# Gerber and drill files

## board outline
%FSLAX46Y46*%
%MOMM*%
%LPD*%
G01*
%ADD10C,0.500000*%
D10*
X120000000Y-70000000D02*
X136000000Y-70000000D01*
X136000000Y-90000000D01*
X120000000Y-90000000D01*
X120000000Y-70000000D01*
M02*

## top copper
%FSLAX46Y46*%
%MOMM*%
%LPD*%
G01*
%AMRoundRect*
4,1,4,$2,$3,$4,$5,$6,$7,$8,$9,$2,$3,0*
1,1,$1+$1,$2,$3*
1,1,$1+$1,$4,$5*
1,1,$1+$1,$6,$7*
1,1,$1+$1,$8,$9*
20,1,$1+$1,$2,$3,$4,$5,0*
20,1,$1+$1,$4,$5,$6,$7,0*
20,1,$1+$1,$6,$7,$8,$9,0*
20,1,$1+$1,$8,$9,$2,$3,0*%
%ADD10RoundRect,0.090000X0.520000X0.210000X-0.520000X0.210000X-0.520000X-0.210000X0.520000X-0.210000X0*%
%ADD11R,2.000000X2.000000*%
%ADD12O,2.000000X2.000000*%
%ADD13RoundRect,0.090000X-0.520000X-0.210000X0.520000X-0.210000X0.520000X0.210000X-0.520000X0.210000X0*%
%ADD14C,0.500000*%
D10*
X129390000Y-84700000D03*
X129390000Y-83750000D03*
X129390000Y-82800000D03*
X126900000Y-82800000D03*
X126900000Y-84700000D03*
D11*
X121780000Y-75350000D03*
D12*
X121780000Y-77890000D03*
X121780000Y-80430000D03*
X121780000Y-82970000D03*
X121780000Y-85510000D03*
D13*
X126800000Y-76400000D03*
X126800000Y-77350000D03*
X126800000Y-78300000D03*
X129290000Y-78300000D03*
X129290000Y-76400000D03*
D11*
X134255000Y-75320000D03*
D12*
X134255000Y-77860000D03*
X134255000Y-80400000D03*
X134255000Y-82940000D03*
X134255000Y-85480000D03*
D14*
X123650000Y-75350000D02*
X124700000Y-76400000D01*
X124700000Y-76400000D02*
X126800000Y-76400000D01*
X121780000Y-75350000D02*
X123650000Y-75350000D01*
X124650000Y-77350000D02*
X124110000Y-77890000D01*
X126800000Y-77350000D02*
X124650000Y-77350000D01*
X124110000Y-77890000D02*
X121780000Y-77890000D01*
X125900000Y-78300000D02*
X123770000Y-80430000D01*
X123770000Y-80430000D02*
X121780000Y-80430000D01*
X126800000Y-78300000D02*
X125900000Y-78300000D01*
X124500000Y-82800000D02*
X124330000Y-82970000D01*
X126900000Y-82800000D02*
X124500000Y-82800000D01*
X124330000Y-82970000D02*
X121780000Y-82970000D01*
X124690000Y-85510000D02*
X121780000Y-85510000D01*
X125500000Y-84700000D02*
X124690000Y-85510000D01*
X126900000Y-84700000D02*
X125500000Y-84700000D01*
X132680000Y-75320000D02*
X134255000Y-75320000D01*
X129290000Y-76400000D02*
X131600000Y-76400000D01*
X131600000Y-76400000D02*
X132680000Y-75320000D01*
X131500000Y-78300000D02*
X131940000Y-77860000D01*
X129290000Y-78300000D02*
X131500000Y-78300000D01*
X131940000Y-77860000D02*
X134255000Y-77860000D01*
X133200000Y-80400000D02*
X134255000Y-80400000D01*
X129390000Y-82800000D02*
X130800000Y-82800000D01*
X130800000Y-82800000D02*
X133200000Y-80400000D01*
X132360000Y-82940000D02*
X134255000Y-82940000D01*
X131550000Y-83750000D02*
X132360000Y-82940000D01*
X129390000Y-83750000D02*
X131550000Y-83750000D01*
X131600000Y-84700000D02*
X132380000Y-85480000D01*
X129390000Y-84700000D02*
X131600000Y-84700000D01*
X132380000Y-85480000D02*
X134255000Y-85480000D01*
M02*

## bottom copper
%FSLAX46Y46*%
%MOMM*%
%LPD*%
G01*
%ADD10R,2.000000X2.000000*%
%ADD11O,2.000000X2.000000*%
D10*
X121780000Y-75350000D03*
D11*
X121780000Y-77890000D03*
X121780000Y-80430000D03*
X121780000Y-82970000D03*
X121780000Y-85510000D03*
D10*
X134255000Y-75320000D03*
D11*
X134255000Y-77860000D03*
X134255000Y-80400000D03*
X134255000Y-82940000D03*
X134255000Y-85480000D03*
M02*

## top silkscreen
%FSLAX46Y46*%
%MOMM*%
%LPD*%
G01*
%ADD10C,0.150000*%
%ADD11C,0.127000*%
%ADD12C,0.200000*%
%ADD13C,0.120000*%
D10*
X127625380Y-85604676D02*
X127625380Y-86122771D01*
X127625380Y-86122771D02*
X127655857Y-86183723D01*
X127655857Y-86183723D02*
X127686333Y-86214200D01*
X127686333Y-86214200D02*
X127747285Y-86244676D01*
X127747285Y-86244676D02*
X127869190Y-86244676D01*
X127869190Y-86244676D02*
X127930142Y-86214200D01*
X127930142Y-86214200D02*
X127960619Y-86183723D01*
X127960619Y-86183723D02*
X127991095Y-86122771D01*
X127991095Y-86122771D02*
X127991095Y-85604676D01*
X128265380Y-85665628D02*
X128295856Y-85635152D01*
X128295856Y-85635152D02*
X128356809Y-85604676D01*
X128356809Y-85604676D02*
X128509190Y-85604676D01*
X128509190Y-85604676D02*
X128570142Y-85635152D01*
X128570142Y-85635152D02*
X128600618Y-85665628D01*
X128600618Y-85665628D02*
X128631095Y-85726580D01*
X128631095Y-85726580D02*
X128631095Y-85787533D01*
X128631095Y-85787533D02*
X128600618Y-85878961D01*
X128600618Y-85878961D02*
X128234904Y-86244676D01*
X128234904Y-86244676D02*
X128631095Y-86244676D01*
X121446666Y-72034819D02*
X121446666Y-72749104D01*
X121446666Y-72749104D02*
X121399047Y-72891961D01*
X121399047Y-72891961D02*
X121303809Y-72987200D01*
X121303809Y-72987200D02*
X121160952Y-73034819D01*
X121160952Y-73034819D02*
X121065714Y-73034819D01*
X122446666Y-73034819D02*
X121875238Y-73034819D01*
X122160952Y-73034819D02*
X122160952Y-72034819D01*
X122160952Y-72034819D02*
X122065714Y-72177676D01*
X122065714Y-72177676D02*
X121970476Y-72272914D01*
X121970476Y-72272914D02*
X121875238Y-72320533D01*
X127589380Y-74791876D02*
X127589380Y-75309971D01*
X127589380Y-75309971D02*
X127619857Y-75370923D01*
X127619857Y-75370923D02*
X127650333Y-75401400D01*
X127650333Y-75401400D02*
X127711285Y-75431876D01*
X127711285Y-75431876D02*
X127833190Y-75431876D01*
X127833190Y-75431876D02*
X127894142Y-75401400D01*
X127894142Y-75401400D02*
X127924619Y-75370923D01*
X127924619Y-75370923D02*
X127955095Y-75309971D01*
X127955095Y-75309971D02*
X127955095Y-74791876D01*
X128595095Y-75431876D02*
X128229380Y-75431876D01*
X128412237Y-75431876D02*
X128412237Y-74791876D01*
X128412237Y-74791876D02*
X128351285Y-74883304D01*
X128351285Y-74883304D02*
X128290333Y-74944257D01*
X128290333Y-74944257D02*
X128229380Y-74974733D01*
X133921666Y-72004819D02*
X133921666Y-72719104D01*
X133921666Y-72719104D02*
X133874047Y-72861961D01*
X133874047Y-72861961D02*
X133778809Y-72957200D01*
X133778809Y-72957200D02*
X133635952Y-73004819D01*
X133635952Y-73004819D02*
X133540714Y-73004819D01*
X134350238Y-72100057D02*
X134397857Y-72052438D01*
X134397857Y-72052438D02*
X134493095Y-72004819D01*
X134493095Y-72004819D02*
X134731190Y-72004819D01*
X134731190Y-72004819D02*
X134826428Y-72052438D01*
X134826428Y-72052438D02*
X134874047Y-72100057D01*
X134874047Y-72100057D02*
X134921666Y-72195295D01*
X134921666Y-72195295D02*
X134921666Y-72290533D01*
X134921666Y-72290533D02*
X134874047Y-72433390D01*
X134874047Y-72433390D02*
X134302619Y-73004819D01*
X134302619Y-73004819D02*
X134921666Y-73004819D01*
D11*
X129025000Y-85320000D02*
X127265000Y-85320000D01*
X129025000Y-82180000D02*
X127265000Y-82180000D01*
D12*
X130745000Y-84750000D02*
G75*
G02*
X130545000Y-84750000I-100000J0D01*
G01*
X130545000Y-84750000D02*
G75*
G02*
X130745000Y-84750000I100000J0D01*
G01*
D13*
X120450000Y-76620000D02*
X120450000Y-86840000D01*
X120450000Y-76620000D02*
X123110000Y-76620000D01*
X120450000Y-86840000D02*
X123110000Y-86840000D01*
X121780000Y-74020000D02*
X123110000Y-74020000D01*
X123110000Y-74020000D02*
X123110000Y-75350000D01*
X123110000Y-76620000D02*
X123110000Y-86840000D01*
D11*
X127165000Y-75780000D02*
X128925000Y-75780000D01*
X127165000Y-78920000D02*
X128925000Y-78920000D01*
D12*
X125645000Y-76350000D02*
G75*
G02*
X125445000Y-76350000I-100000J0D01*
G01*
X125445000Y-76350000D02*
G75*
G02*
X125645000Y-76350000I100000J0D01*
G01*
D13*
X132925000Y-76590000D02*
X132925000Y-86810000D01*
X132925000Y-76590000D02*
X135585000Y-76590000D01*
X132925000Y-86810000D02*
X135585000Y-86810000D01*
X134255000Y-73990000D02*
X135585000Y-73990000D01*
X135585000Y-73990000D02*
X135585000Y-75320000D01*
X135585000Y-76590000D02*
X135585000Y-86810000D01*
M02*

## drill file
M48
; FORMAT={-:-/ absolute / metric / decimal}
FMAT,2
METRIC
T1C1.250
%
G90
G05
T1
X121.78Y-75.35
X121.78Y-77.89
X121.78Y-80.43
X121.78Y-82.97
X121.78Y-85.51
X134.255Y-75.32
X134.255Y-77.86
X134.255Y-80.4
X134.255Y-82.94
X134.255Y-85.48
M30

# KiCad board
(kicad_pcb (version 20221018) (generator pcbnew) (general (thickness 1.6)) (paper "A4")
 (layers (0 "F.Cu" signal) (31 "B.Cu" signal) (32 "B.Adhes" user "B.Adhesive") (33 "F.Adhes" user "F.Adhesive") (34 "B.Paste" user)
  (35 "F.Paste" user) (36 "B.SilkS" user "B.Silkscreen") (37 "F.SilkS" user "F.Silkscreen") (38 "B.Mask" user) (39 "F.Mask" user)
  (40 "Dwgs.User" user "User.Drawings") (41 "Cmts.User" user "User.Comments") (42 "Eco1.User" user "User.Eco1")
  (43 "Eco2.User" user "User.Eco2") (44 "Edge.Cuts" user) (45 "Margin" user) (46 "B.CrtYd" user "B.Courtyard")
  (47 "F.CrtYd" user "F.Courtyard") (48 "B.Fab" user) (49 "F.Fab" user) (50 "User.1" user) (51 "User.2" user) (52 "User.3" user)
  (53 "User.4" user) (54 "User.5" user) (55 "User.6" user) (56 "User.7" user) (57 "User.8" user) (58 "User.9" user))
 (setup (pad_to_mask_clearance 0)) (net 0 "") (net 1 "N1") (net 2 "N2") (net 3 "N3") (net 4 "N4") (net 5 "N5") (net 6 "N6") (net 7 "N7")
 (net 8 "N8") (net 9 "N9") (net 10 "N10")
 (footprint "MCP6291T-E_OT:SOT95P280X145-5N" (layer "F.Cu") (at 128.145 83.75 180)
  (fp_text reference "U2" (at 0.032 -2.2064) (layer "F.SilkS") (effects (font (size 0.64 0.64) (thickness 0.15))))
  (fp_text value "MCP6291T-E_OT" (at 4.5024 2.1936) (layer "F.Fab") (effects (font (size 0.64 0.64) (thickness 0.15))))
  (fp_line (start -0.88 -1.57) (end 0.88 -1.57) (stroke (width 0.127) (type solid)) (layer "F.SilkS"))
  (fp_line (start -0.88 1.57) (end 0.88 1.57) (stroke (width 0.127) (type solid)) (layer "F.SilkS"))
  (fp_circle (center -2.5 -1) (end -2.4 -1) (stroke (width 0.2) (type solid)) (fill none) (layer "F.SilkS"))
  (pad "1" smd roundrect (at -1.245 -0.95 180) (size 1.22 0.6) (layers "F.Cu" "F.Paste" "F.Mask") (roundrect_rratio 0.15) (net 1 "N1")
   (solder_mask_margin 0.102))
  (pad "2" smd roundrect (at -1.245 0 180) (size 1.22 0.6) (layers "F.Cu" "F.Paste" "F.Mask") (roundrect_rratio 0.15) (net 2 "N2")
   (solder_mask_margin 0.102))
  (pad "3" smd roundrect (at -1.245 0.95 180) (size 1.22 0.6) (layers "F.Cu" "F.Paste" "F.Mask") (roundrect_rratio 0.15) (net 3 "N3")
   (solder_mask_margin 0.102))
  (pad "4" smd roundrect (at 1.245 0.95 180) (size 1.22 0.6) (layers "F.Cu" "F.Paste" "F.Mask") (roundrect_rratio 0.15) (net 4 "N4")
   (solder_mask_margin 0.102))
  (pad "5" smd roundrect (at 1.245 -0.95 180) (size 1.22 0.6) (layers "F.Cu" "F.Paste" "F.Mask") (roundrect_rratio 0.15) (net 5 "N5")
   (solder_mask_margin 0.102)))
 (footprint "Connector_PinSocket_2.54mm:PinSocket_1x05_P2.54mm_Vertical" (layer "F.Cu") (at 121.78 75.35)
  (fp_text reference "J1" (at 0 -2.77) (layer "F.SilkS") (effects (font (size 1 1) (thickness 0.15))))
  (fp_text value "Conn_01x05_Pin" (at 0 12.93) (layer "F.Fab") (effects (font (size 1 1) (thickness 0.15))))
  (fp_line (start -1.33 1.27) (end -1.33 11.49) (stroke (width 0.12) (type solid)) (layer "F.SilkS"))
  (fp_line (start -1.33 1.27) (end 1.33 1.27) (stroke (width 0.12) (type solid)) (layer "F.SilkS"))
  (fp_line (start -1.33 11.49) (end 1.33 11.49) (stroke (width 0.12) (type solid)) (layer "F.SilkS"))
  (fp_line (start 0 -1.33) (end 1.33 -1.33) (stroke (width 0.12) (type solid)) (layer "F.SilkS"))
  (fp_line (start 1.33 -1.33) (end 1.33 0) (stroke (width 0.12) (type solid)) (layer "F.SilkS"))
  (fp_line (start 1.33 1.27) (end 1.33 11.49) (stroke (width 0.12) (type solid)) (layer "F.SilkS"))
  (pad "1" thru_hole rect (at 0 0) (size 2 2) (drill 1.25) (layers "*.Cu" "*.Mask") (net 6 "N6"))
  (pad "2" thru_hole oval (at 0 2.54) (size 2 2) (drill 1.25) (layers "*.Cu" "*.Mask") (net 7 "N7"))
  (pad "3" thru_hole oval (at 0 5.08) (size 2 2) (drill 1.25) (layers "*.Cu" "*.Mask") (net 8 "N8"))
  (pad "4" thru_hole oval (at 0 7.62) (size 2 2) (drill 1.25) (layers "*.Cu" "*.Mask") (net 4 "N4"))
  (pad "5" thru_hole oval (at 0 10.16) (size 2 2) (drill 1.25) (layers "*.Cu" "*.Mask") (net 5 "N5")))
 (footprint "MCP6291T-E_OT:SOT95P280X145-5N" (layer "F.Cu") (at 128.045 77.35)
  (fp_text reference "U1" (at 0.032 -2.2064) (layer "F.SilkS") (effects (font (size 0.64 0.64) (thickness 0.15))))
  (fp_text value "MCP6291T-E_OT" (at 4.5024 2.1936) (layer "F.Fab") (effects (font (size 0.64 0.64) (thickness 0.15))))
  (fp_line (start -0.88 -1.57) (end 0.88 -1.57) (stroke (width 0.127) (type solid)) (layer "F.SilkS"))
  (fp_line (start -0.88 1.57) (end 0.88 1.57) (stroke (width 0.127) (type solid)) (layer "F.SilkS"))
  (fp_circle (center -2.5 -1) (end -2.4 -1) (stroke (width 0.2) (type solid)) (fill none) (layer "F.SilkS"))
  (pad "1" smd roundrect (at -1.245 -0.95) (size 1.22 0.6) (layers "F.Cu" "F.Paste" "F.Mask") (roundrect_rratio 0.15) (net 6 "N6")
   (solder_mask_margin 0.102))
  (pad "2" smd roundrect (at -1.245 0) (size 1.22 0.6) (layers "F.Cu" "F.Paste" "F.Mask") (roundrect_rratio 0.15) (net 7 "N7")
   (solder_mask_margin 0.102))
  (pad "3" smd roundrect (at -1.245 0.95) (size 1.22 0.6) (layers "F.Cu" "F.Paste" "F.Mask") (roundrect_rratio 0.15) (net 8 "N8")
   (solder_mask_margin 0.102))
  (pad "4" smd roundrect (at 1.245 0.95) (size 1.22 0.6) (layers "F.Cu" "F.Paste" "F.Mask") (roundrect_rratio 0.15) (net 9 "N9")
   (solder_mask_margin 0.102))
  (pad "5" smd roundrect (at 1.245 -0.95) (size 1.22 0.6) (layers "F.Cu" "F.Paste" "F.Mask") (roundrect_rratio 0.15) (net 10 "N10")
   (solder_mask_margin 0.102)))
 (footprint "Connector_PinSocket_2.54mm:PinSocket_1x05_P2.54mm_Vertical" (layer "F.Cu") (at 134.255 75.32)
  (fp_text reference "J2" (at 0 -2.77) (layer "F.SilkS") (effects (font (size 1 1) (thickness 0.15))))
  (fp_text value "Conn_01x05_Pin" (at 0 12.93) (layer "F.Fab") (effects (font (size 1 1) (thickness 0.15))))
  (fp_line (start -1.33 1.27) (end -1.33 11.49) (stroke (width 0.12) (type solid)) (layer "F.SilkS"))
  (fp_line (start -1.33 1.27) (end 1.33 1.27) (stroke (width 0.12) (type solid)) (layer "F.SilkS"))
  (fp_line (start -1.33 11.49) (end 1.33 11.49) (stroke (width 0.12) (type solid)) (layer "F.SilkS"))
  (fp_line (start 0 -1.33) (end 1.33 -1.33) (stroke (width 0.12) (type solid)) (layer "F.SilkS"))
  (fp_line (start 1.33 -1.33) (end 1.33 0) (stroke (width 0.12) (type solid)) (layer "F.SilkS"))
  (fp_line (start 1.33 1.27) (end 1.33 11.49) (stroke (width 0.12) (type solid)) (layer "F.SilkS"))
  (pad "1" thru_hole rect (at 0 0) (size 2 2) (drill 1.25) (layers "*.Cu" "*.Mask") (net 10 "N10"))
  (pad "2" thru_hole oval (at 0 2.54) (size 2 2) (drill 1.25) (layers "*.Cu" "*.Mask") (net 9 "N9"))
  (pad "3" thru_hole oval (at 0 5.08) (size 2 2) (drill 1.25) (layers "*.Cu" "*.Mask") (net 3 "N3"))
  (pad "4" thru_hole oval (at 0 7.62) (size 2 2) (drill 1.25) (layers "*.Cu" "*.Mask") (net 2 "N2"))
  (pad "5" thru_hole oval (at 0 10.16) (size 2 2) (drill 1.25) (layers "*.Cu" "*.Mask") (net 1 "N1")))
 (gr_rect (start 120 70) (end 136 90) (stroke (width 0.5) (type default)) (fill none) (layer "Edge.Cuts"))
 (gr_rect (start 136 88.6) (end 136 88.6) (stroke (width 0.1) (type default)) (fill none) (layer "Edge.Cuts"))
 (segment (start 123.65 75.35) (end 124.7 76.4) (width 0.5) (layer "F.Cu") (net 6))
 (segment (start 124.7 76.4) (end 126.8 76.4) (width 0.5) (layer "F.Cu") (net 6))
 (segment (start 121.78 75.35) (end 123.65 75.35) (width 0.5) (layer "F.Cu") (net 6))
 (segment (start 124.65 77.35) (end 124.11 77.89) (width 0.5) (layer "F.Cu") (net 7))
 (segment (start 126.8 77.35) (end 124.65 77.35) (width 0.5) (layer "F.Cu") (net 7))
 (segment (start 124.11 77.89) (end 121.78 77.89) (width 0.5) (layer "F.Cu") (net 7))
 (segment (start 125.9 78.3) (end 123.77 80.43) (width 0.5) (layer "F.Cu") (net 8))
 (segment (start 123.77 80.43) (end 121.78 80.43) (width 0.5) (layer "F.Cu") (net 8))
 (segment (start 126.8 78.3) (end 125.9 78.3) (width 0.5) (layer "F.Cu") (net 8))
 (segment (start 124.5 82.8) (end 124.33 82.97) (width 0.5) (layer "F.Cu") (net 4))
 (segment (start 126.9 82.8) (end 124.5 82.8) (width 0.5) (layer "F.Cu") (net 4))
 (segment (start 124.33 82.97) (end 121.78 82.97) (width 0.5) (layer "F.Cu") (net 4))
 (segment (start 124.69 85.51) (end 121.78 85.51) (width 0.5) (layer "F.Cu") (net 5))
 (segment (start 125.5 84.7) (end 124.69 85.51) (width 0.5) (layer "F.Cu") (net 5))
 (segment (start 126.9 84.7) (end 125.5 84.7) (width 0.5) (layer "F.Cu") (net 5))
 (segment (start 132.68 75.32) (end 134.255 75.32) (width 0.5) (layer "F.Cu") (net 10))
 (segment (start 129.29 76.4) (end 131.6 76.4) (width 0.5) (layer "F.Cu") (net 10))
 (segment (start 131.6 76.4) (end 132.68 75.32) (width 0.5) (layer "F.Cu") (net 10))
 (segment (start 131.5 78.3) (end 131.94 77.86) (width 0.5) (layer "F.Cu") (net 9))
 (segment (start 129.29 78.3) (end 131.5 78.3) (width 0.5) (layer "F.Cu") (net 9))
 (segment (start 131.94 77.86) (end 134.255 77.86) (width 0.5) (layer "F.Cu") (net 9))
 (segment (start 133.2 80.4) (end 134.255 80.4) (width 0.5) (layer "F.Cu") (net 3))
 (segment (start 129.39 82.8) (end 130.8 82.8) (width 0.5) (layer "F.Cu") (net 3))
 (segment (start 130.8 82.8) (end 133.2 80.4) (width 0.5) (layer "F.Cu") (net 3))
 (segment (start 132.36 82.94) (end 134.255 82.94) (width 0.5) (layer "F.Cu") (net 2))
 (segment (start 131.55 83.75) (end 132.36 82.94) (width 0.5) (layer "F.Cu") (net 2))
 (segment (start 129.39 83.75) (end 131.55 83.75) (width 0.5) (layer "F.Cu") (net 2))
 (segment (start 131.6 84.7) (end 132.38 85.48) (width 0.5) (layer "F.Cu") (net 1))
 (segment (start 129.39 84.7) (end 131.6 84.7) (width 0.5) (layer "F.Cu") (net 1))
 (segment (start 132.38 85.48) (end 134.255 85.48) (width 0.5) (layer "F.Cu") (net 1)))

